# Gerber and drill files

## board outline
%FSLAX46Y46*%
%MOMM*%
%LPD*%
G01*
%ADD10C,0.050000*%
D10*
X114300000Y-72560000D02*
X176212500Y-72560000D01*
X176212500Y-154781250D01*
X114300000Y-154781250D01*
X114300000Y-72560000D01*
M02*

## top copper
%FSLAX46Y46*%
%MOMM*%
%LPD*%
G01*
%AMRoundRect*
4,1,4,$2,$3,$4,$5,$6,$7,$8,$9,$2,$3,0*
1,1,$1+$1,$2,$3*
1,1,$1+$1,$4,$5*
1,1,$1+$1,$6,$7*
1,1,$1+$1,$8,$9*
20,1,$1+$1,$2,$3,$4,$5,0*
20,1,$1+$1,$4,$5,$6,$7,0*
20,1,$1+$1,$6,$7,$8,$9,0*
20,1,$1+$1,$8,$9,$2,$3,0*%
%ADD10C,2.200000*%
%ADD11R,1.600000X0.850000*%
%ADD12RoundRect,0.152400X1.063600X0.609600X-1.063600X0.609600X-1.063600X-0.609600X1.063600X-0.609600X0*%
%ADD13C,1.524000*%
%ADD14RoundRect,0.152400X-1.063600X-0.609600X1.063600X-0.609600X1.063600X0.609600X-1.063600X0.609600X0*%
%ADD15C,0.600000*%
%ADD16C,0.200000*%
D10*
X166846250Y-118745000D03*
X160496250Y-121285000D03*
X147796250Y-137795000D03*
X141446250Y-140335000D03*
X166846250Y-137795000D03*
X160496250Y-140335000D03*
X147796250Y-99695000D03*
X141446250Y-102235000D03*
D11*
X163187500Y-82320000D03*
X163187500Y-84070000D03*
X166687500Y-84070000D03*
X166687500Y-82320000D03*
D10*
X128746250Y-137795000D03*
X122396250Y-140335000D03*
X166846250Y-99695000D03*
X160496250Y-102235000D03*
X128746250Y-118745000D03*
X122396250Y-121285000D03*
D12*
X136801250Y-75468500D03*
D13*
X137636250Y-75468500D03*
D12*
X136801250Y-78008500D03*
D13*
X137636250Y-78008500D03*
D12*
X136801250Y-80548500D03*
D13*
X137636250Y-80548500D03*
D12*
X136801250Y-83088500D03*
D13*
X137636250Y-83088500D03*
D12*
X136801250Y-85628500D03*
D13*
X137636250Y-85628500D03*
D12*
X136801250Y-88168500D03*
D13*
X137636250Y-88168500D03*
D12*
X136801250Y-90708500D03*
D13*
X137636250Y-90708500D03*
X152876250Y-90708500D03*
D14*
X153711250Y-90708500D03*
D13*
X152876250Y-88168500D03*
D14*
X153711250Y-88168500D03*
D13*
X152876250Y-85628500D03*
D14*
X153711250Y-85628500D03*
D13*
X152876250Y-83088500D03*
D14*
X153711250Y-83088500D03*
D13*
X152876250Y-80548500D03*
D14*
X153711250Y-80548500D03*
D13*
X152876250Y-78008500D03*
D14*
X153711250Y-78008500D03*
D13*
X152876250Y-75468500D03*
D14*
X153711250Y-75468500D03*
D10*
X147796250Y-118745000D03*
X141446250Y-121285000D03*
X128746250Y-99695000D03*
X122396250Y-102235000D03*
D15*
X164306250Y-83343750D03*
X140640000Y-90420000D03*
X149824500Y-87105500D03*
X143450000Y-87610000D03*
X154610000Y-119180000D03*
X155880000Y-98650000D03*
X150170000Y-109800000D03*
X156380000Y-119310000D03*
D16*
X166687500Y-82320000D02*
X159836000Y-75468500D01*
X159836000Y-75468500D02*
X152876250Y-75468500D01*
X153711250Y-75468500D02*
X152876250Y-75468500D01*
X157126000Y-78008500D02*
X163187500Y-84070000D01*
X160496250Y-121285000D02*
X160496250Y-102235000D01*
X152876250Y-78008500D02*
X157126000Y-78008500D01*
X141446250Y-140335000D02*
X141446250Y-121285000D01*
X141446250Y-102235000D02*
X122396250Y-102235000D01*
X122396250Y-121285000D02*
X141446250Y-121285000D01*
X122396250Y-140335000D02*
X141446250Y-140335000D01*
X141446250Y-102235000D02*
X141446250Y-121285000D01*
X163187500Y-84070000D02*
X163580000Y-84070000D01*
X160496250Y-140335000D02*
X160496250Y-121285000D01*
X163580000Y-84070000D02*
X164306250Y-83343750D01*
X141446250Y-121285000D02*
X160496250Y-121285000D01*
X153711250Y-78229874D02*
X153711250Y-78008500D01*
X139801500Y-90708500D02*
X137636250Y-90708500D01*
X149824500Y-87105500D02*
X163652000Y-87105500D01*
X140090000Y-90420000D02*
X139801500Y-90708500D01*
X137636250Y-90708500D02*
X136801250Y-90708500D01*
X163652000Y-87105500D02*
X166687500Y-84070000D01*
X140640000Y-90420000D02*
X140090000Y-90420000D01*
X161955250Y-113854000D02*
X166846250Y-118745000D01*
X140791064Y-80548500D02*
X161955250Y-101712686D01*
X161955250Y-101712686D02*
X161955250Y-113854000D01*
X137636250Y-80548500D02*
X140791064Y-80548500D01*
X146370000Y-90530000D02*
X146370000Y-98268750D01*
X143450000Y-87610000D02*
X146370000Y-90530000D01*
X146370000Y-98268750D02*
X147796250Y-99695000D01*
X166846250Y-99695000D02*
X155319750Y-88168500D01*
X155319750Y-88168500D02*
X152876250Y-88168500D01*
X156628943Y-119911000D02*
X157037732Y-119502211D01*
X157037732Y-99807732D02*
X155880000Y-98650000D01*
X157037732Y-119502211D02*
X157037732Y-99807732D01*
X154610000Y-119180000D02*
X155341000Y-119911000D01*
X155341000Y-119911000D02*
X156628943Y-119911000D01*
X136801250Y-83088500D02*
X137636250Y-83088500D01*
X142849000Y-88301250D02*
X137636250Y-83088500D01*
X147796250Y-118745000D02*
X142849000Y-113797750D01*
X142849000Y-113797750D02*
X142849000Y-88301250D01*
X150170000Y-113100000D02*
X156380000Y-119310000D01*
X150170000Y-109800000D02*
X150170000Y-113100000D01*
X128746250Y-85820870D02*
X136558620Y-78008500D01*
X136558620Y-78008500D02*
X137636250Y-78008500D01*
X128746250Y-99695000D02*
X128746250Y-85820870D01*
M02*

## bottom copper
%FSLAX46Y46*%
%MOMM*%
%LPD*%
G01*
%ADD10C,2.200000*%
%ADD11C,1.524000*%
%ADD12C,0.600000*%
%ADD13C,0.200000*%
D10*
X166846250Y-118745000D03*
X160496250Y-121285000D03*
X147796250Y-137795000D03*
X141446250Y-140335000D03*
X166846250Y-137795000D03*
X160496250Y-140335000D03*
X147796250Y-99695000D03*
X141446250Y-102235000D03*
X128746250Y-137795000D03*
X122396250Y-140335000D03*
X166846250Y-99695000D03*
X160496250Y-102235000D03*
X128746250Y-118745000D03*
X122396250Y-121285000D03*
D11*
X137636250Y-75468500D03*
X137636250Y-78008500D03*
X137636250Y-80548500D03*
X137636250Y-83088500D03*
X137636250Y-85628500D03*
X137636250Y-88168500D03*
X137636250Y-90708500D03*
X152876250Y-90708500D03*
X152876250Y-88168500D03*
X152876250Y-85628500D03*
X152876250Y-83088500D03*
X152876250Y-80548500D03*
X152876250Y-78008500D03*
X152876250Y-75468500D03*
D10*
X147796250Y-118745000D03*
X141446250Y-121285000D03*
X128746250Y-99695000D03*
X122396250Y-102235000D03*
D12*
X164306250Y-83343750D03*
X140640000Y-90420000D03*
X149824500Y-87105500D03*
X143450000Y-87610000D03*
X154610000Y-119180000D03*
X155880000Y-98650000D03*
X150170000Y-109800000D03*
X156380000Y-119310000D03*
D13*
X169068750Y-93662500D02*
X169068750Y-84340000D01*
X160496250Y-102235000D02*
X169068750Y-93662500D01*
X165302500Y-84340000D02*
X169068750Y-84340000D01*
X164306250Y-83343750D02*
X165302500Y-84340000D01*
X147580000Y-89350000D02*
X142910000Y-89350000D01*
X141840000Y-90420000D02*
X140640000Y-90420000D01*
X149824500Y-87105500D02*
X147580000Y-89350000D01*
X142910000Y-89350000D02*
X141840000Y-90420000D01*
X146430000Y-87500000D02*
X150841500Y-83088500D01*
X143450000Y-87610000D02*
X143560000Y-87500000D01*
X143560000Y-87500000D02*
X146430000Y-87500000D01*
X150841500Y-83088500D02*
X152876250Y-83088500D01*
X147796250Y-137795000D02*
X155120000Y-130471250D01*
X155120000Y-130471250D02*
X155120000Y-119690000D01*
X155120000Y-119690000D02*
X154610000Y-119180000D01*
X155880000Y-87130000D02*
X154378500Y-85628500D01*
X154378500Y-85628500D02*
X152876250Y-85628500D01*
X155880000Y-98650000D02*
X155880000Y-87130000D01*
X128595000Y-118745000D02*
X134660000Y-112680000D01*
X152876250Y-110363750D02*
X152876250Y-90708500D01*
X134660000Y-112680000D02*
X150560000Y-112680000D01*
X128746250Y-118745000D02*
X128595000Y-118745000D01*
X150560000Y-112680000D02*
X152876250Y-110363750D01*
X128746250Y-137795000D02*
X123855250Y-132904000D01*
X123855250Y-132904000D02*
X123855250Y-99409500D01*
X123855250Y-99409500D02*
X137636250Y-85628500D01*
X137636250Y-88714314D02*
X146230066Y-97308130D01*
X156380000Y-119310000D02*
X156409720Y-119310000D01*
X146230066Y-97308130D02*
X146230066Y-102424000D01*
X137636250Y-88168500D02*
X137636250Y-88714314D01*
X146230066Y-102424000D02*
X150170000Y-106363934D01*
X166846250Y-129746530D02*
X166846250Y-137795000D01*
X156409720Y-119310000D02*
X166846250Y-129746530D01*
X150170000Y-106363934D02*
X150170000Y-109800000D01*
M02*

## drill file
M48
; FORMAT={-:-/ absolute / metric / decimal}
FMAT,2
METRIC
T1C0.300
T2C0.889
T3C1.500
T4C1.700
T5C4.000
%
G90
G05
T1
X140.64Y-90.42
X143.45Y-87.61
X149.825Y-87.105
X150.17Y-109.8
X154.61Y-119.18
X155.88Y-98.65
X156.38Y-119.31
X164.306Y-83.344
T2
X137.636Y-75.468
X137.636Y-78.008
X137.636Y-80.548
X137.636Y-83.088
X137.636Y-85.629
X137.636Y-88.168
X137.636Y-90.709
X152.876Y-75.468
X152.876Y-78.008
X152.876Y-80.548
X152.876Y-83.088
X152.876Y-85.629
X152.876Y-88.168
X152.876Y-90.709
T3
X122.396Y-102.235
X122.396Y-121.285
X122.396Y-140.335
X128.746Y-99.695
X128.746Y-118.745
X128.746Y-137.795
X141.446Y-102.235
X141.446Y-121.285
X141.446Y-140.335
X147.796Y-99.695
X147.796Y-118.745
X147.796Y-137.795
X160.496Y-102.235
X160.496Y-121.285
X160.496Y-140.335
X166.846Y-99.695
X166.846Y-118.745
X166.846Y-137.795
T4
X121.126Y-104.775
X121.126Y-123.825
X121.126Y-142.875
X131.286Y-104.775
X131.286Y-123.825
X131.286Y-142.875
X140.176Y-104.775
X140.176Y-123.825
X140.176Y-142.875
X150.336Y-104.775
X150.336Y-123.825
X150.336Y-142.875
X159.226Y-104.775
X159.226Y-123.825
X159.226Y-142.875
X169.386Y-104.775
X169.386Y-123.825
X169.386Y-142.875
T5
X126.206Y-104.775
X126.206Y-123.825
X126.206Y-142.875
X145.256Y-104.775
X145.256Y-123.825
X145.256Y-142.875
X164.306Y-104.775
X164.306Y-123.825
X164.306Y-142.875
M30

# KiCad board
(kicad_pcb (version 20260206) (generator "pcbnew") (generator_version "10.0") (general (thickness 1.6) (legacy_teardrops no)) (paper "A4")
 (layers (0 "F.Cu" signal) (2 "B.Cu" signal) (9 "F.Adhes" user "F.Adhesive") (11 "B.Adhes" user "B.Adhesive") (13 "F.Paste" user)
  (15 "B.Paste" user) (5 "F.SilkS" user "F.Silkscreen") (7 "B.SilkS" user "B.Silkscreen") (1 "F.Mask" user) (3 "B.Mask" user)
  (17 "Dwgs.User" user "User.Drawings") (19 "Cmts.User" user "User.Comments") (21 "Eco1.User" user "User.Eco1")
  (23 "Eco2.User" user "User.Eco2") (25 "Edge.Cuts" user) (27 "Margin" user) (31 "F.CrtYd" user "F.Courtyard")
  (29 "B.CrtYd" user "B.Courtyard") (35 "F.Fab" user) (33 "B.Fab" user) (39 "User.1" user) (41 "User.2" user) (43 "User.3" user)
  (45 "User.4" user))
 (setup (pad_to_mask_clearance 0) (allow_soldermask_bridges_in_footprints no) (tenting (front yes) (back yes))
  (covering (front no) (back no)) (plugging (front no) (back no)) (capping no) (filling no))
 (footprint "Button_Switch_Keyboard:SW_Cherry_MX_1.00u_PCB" (layer "F.Cu") (at 166.84625 118.745)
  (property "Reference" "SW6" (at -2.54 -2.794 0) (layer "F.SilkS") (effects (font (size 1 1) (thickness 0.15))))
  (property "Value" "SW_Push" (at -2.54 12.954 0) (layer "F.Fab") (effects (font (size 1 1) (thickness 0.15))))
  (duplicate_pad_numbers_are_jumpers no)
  (pad "" np_thru_hole circle (at -7.62 5.08) (size 1.7 1.7) (drill 1.7) (layers "*.Cu" "*.Mask"))
  (pad "" np_thru_hole circle (at -2.54 5.08) (size 4 4) (drill 4) (layers "*.Cu" "*.Mask"))
  (pad "" np_thru_hole circle (at 2.54 5.08) (size 1.7 1.7) (drill 1.7) (layers "*.Cu" "*.Mask"))
  (pad "1" thru_hole circle (at 0 0) (size 2.2 2.2) (drill 1.5) (layers "*.Cu" "*.Mask") (remove_unused_layers no)
   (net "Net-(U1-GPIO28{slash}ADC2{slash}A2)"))
  (pad "2" thru_hole circle (at -6.35 2.54) (size 2.2 2.2) (drill 1.5) (layers "*.Cu" "*.Mask") (remove_unused_layers no) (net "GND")))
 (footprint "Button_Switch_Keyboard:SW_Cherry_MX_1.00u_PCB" (layer "F.Cu") (at 147.79625 137.795)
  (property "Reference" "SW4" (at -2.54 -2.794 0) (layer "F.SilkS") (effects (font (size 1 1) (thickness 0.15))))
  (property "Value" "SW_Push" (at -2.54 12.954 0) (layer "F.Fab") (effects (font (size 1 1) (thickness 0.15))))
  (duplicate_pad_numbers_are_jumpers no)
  (pad "" np_thru_hole circle (at -7.62 5.08) (size 1.7 1.7) (drill 1.7) (layers "*.Cu" "*.Mask"))
  (pad "" np_thru_hole circle (at -2.54 5.08) (size 4 4) (drill 4) (layers "*.Cu" "*.Mask"))
  (pad "" np_thru_hole circle (at 2.54 5.08) (size 1.7 1.7) (drill 1.7) (layers "*.Cu" "*.Mask"))
  (pad "1" thru_hole circle (at 0 0) (size 2.2 2.2) (drill 1.5) (layers "*.Cu" "*.Mask") (remove_unused_layers no)
   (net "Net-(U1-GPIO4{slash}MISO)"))
  (pad "2" thru_hole circle (at -6.35 2.54) (size 2.2 2.2) (drill 1.5) (layers "*.Cu" "*.Mask") (remove_unused_layers no) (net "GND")))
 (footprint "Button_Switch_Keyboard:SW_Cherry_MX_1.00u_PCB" (layer "F.Cu") (at 166.84625 137.795)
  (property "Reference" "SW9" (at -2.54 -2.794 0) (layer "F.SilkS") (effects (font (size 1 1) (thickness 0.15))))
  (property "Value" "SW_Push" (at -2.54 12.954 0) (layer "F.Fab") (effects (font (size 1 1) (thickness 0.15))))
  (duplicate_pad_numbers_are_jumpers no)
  (pad "" np_thru_hole circle (at -7.62 5.08) (size 1.7 1.7) (drill 1.7) (layers "*.Cu" "*.Mask"))
  (pad "" np_thru_hole circle (at -2.54 5.08) (size 4 4) (drill 4) (layers "*.Cu" "*.Mask"))
  (pad "" np_thru_hole circle (at 2.54 5.08) (size 1.7 1.7) (drill 1.7) (layers "*.Cu" "*.Mask"))
  (pad "1" thru_hole circle (at 0 0) (size 2.2 2.2) (drill 1.5) (layers "*.Cu" "*.Mask") (remove_unused_layers no)
   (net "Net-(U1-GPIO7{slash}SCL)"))
  (pad "2" thru_hole circle (at -6.35 2.54) (size 2.2 2.2) (drill 1.5) (layers "*.Cu" "*.Mask") (remove_unused_layers no) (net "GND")))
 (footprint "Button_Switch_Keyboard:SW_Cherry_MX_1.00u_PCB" (layer "F.Cu") (at 147.79625 99.695)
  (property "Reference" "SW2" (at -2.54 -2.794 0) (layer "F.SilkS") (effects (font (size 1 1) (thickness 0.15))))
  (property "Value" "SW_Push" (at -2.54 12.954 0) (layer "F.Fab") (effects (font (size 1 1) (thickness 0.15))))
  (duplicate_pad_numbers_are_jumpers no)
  (pad "" np_thru_hole circle (at -7.62 5.08) (size 1.7 1.7) (drill 1.7) (layers "*.Cu" "*.Mask"))
  (pad "" np_thru_hole circle (at -2.54 5.08) (size 4 4) (drill 4) (layers "*.Cu" "*.Mask"))
  (pad "" np_thru_hole circle (at 2.54 5.08) (size 1.7 1.7) (drill 1.7) (layers "*.Cu" "*.Mask"))
  (pad "1" thru_hole circle (at 0 0) (size 2.2 2.2) (drill 1.5) (layers "*.Cu" "*.Mask") (remove_unused_layers no)
   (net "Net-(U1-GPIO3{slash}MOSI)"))
  (pad "2" thru_hole circle (at -6.35 2.54) (size 2.2 2.2) (drill 1.5) (layers "*.Cu" "*.Mask") (remove_unused_layers no) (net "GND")))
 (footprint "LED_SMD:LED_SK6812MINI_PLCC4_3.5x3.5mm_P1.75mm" (layer "F.Cu") (at 164.9375 83.195)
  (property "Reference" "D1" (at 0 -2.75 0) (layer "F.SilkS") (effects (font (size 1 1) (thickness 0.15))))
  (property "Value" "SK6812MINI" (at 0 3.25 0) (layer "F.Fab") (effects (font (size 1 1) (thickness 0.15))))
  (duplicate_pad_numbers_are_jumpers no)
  (pad "1" smd rect (at -1.75 -0.875) (size 1.6 0.85) (layers "F.Cu" "F.Mask" "F.Paste") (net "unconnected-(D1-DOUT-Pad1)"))
  (pad "2" smd rect (at -1.75 0.875) (size 1.6 0.85) (layers "F.Cu" "F.Mask" "F.Paste") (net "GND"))
  (pad "3" smd rect (at 1.75 0.875) (size 1.6 0.85) (layers "F.Cu" "F.Mask" "F.Paste") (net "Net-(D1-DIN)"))
  (pad "4" smd rect (at 1.75 -0.875) (size 1.6 0.85) (layers "F.Cu" "F.Mask" "F.Paste") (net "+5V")))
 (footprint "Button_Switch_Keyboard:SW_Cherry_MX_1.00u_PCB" (layer "F.Cu") (at 128.74625 137.795)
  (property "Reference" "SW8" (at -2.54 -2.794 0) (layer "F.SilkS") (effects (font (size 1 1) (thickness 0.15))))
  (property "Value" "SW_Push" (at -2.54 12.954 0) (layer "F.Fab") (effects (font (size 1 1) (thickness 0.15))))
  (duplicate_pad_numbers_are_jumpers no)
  (pad "" np_thru_hole circle (at -7.62 5.08) (size 1.7 1.7) (drill 1.7) (layers "*.Cu" "*.Mask"))
  (pad "" np_thru_hole circle (at -2.54 5.08) (size 4 4) (drill 4) (layers "*.Cu" "*.Mask"))
  (pad "" np_thru_hole circle (at 2.54 5.08) (size 1.7 1.7) (drill 1.7) (layers "*.Cu" "*.Mask"))
  (pad "1" thru_hole circle (at 0 0) (size 2.2 2.2) (drill 1.5) (layers "*.Cu" "*.Mask") (remove_unused_layers no)
   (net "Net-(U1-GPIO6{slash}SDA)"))
  (pad "2" thru_hole circle (at -6.35 2.54) (size 2.2 2.2) (drill 1.5) (layers "*.Cu" "*.Mask") (remove_unused_layers no) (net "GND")))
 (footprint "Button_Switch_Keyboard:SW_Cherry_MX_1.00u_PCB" (layer "F.Cu") (at 166.84625 99.695)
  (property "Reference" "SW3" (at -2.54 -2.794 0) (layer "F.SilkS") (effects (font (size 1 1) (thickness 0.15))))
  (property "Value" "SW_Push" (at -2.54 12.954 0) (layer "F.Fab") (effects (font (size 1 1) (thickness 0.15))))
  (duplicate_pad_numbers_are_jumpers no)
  (pad "" np_thru_hole circle (at -7.62 5.08) (size 1.7 1.7) (drill 1.7) (layers "*.Cu" "*.Mask"))
  (pad "" np_thru_hole circle (at -2.54 5.08) (size 4 4) (drill 4) (layers "*.Cu" "*.Mask"))
  (pad "" np_thru_hole circle (at 2.54 5.08) (size 1.7 1.7) (drill 1.7) (layers "*.Cu" "*.Mask"))
  (pad "1" thru_hole circle (at 0 0) (size 2.2 2.2) (drill 1.5) (layers "*.Cu" "*.Mask") (remove_unused_layers no)
   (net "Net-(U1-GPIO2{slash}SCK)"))
  (pad "2" thru_hole circle (at -6.35 2.54) (size 2.2 2.2) (drill 1.5) (layers "*.Cu" "*.Mask") (remove_unused_layers no) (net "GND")))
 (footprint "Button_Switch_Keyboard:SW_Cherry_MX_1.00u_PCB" (layer "F.Cu") (at 128.74625 118.745)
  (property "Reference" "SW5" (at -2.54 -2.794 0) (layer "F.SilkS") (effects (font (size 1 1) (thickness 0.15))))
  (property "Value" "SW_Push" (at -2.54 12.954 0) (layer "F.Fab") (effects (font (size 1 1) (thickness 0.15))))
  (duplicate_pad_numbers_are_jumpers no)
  (pad "" np_thru_hole circle (at -7.62 5.08) (size 1.7 1.7) (drill 1.7) (layers "*.Cu" "*.Mask"))
  (pad "" np_thru_hole circle (at -2.54 5.08) (size 4 4) (drill 4) (layers "*.Cu" "*.Mask"))
  (pad "" np_thru_hole circle (at 2.54 5.08) (size 1.7 1.7) (drill 1.7) (layers "*.Cu" "*.Mask"))
  (pad "1" thru_hole circle (at 0 0) (size 2.2 2.2) (drill 1.5) (layers "*.Cu" "*.Mask") (remove_unused_layers no)
   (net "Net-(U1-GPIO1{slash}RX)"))
  (pad "2" thru_hole circle (at -6.35 2.54) (size 2.2 2.2) (drill 1.5) (layers "*.Cu" "*.Mask") (remove_unused_layers no) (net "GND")))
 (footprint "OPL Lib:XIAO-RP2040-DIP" (layer "F.Cu") (at 145.25625 83.0885)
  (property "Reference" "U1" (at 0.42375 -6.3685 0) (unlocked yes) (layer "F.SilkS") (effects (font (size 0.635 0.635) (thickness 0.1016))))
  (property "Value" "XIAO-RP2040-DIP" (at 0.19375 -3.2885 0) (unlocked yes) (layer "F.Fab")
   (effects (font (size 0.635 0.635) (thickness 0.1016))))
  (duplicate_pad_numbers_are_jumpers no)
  (pad "1" smd roundrect (at -8.455 -7.62 180) (size 2.432 1.524) (layers "F.Cu" "F.Mask") (roundrect_rratio 0.1)
   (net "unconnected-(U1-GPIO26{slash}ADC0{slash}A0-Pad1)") (thermal_bridge_angle 45))
  (pad "1" thru_hole circle (at -7.62 -7.62 180) (size 1.524 1.524) (drill 0.889) (layers "*.Cu" "*.Mask") (remove_unused_layers no)
   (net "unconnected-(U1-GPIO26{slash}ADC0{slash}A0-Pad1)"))
  (pad "2" smd roundrect (at -8.455 -5.08 180) (size 2.432 1.524) (layers "F.Cu" "F.Mask") (roundrect_rratio 0.1)
   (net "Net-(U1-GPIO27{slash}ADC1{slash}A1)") (thermal_bridge_angle 45))
  (pad "2" thru_hole circle (at -7.62 -5.08 180) (size 1.524 1.524) (drill 0.889) (layers "*.Cu" "*.Mask") (remove_unused_layers no)
   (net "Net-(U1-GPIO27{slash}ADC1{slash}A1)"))
  (pad "3" smd roundrect (at -8.455 -2.54 180) (size 2.432 1.524) (layers "F.Cu" "F.Mask") (roundrect_rratio 0.1)
   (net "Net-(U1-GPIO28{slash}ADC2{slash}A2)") (thermal_bridge_angle 45))
  (pad "3" thru_hole circle (at -7.62 -2.54 180) (size 1.524 1.524) (drill 0.889) (layers "*.Cu" "*.Mask") (remove_unused_layers no)
   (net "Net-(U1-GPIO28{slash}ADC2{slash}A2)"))
  (pad "4" smd roundrect (at -8.455 0 180) (size 2.432 1.524) (layers "F.Cu" "F.Mask") (roundrect_rratio 0.1)
   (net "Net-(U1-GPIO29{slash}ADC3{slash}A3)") (thermal_bridge_angle 45))
  (pad "4" thru_hole circle (at -7.62 0 180) (size 1.524 1.524) (drill 0.889) (layers "*.Cu" "*.Mask") (remove_unused_layers no)
   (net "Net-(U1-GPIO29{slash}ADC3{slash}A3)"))
  (pad "5" smd roundrect (at -8.455 2.54 180) (size 2.432 1.524) (layers "F.Cu" "F.Mask") (roundrect_rratio 0.1)
   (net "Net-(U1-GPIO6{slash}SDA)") (thermal_bridge_angle 45))
  (pad "5" thru_hole circle (at -7.62 2.54 180) (size 1.524 1.524) (drill 0.889) (layers "*.Cu" "*.Mask") (remove_unused_layers no)
   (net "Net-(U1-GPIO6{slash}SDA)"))
  (pad "6" smd roundrect (at -8.455 5.08 180) (size 2.432 1.524) (layers "F.Cu" "F.Mask") (roundrect_rratio 0.1)
   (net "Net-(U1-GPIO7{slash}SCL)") (thermal_bridge_angle 45))
  (pad "6" thru_hole circle (at -7.62 5.08 180) (size 1.524 1.524) (drill 0.889) (layers "*.Cu" "*.Mask") (remove_unused_layers no)
   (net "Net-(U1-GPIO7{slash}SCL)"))
  (pad "7" smd roundrect (at -8.455 7.62 180) (size 2.432 1.524) (layers "F.Cu" "F.Mask") (roundrect_rratio 0.1) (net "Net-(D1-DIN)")
   (thermal_bridge_angle 45))
  (pad "7" thru_hole circle (at -7.62 7.62 180) (size 1.524 1.524) (drill 0.889) (layers "*.Cu" "*.Mask") (remove_unused_layers no)
   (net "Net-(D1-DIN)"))
  (pad "8" thru_hole circle (at 7.62 7.62) (size 1.524 1.524) (drill 0.889) (layers "*.Cu" "*.Mask") (remove_unused_layers no)
   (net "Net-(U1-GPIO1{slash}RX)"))
  (pad "8" smd roundrect (at 8.455 7.62) (size 2.432 1.524) (layers "F.Cu" "F.Mask") (roundrect_rratio 0.1) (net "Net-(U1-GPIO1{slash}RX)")
   (thermal_bridge_angle 45))
  (pad "9" thru_hole circle (at 7.62 5.08) (size 1.524 1.524) (drill 0.889) (layers "*.Cu" "*.Mask") (remove_unused_layers no)
   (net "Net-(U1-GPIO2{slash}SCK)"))
  (pad "9" smd roundrect (at 8.455 5.08) (size 2.432 1.524) (layers "F.Cu" "F.Mask") (roundrect_rratio 0.1) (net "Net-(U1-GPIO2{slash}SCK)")
   (thermal_bridge_angle 45))
  (pad "10" thru_hole circle (at 7.62 2.54) (size 1.524 1.524) (drill 0.889) (layers "*.Cu" "*.Mask") (remove_unused_layers no)
   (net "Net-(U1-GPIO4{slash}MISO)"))
  (pad "10" smd roundrect (at 8.455 2.54) (size 2.432 1.524) (layers "F.Cu" "F.Mask") (roundrect_rratio 0.1)
   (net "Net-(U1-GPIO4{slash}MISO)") (thermal_bridge_angle 45))
  (pad "11" thru_hole circle (at 7.62 0) (size 1.524 1.524) (drill 0.889) (layers "*.Cu" "*.Mask") (remove_unused_layers no)
   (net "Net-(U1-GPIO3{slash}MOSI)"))
  (pad "11" smd roundrect (at 8.455 0) (size 2.432 1.524) (layers "F.Cu" "F.Mask") (roundrect_rratio 0.1) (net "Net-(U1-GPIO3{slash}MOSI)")
   (thermal_bridge_angle 45))
  (pad "12" thru_hole circle (at 7.62 -2.54) (size 1.524 1.524) (drill 0.889) (layers "*.Cu" "*.Mask") (remove_unused_layers no)
   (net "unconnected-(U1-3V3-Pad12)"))
  (pad "12" smd roundrect (at 8.455 -2.54) (size 2.432 1.524) (layers "F.Cu" "F.Mask") (roundrect_rratio 0.1)
   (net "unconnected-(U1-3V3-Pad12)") (thermal_bridge_angle 45))
  (pad "13" thru_hole circle (at 7.62 -5.08) (size 1.524 1.524) (drill 0.889) (layers "*.Cu" "*.Mask") (remove_unused_layers no) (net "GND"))
  (pad "13" smd roundrect (at 8.455 -5.08) (size 2.432 1.524) (layers "F.Cu" "F.Mask") (roundrect_rratio 0.1) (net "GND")
   (thermal_bridge_angle 45))
  (pad "14" thru_hole circle (at 7.62 -7.62) (size 1.524 1.524) (drill 0.889) (layers "*.Cu" "*.Mask") (remove_unused_layers no) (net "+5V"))
  (pad "14" smd roundrect (at 8.455 -7.62) (size 2.432 1.524) (layers "F.Cu" "F.Mask") (roundrect_rratio 0.1) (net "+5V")
   (thermal_bridge_angle 45)))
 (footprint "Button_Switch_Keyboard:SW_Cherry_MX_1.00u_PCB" (layer "F.Cu") (at 147.79625 118.745)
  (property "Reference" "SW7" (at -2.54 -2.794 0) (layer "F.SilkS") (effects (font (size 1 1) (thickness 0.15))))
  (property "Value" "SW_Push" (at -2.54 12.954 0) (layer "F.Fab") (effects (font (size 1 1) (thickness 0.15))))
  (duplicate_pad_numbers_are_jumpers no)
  (pad "" np_thru_hole circle (at -7.62 5.08) (size 1.7 1.7) (drill 1.7) (layers "*.Cu" "*.Mask"))
  (pad "" np_thru_hole circle (at -2.54 5.08) (size 4 4) (drill 4) (layers "*.Cu" "*.Mask"))
  (pad "" np_thru_hole circle (at 2.54 5.08) (size 1.7 1.7) (drill 1.7) (layers "*.Cu" "*.Mask"))
  (pad "1" thru_hole circle (at 0 0) (size 2.2 2.2) (drill 1.5) (layers "*.Cu" "*.Mask") (remove_unused_layers no)
   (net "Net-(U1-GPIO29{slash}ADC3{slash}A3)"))
  (pad "2" thru_hole circle (at -6.35 2.54) (size 2.2 2.2) (drill 1.5) (layers "*.Cu" "*.Mask") (remove_unused_layers no) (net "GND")))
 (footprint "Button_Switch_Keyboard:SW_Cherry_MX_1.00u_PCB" (layer "F.Cu") (at 128.74625 99.695)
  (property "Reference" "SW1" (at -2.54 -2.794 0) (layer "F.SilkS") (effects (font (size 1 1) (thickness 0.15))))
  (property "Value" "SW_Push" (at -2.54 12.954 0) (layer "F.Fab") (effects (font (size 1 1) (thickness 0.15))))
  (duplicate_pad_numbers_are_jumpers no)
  (pad "" np_thru_hole circle (at -7.62 5.08) (size 1.7 1.7) (drill 1.7) (layers "*.Cu" "*.Mask"))
  (pad "" np_thru_hole circle (at -2.54 5.08) (size 4 4) (drill 4) (layers "*.Cu" "*.Mask"))
  (pad "" np_thru_hole circle (at 2.54 5.08) (size 1.7 1.7) (drill 1.7) (layers "*.Cu" "*.Mask"))
  (pad "1" thru_hole circle (at 0 0) (size 2.2 2.2) (drill 1.5) (layers "*.Cu" "*.Mask") (remove_unused_layers no)
   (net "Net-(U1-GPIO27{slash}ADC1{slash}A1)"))
  (pad "2" thru_hole circle (at -6.35 2.54) (size 2.2 2.2) (drill 1.5) (layers "*.Cu" "*.Mask") (remove_unused_layers no) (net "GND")))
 (gr_rect (start 114.3 72.56) (end 176.2125 154.78125) (stroke (width 0.05) (type default)) (fill no) (layer "Edge.Cuts"))
 (segment (start 166.6875 82.32) (end 159.836 75.4685) (width 0.2) (layer "F.Cu") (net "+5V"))
 (segment (start 159.836 75.4685) (end 152.87625 75.4685) (width 0.2) (layer "F.Cu") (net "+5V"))
 (segment (start 153.71125 75.4685) (end 152.87625 75.4685) (width 0.2) (layer "F.Cu") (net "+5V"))
 (segment (start 157.126 78.0085) (end 163.1875 84.07) (width 0.2) (layer "F.Cu") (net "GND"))
 (segment (start 160.49625 121.285) (end 160.49625 102.235) (width 0.2) (layer "F.Cu") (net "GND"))
 (segment (start 152.87625 78.0085) (end 157.126 78.0085) (width 0.2) (layer "F.Cu") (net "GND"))
 (segment (start 141.44625 140.335) (end 141.44625 121.285) (width 0.2) (layer "F.Cu") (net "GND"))
 (segment (start 141.44625 102.235) (end 122.39625 102.235) (width 0.2) (layer "F.Cu") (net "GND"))
 (segment (start 122.39625 121.285) (end 141.44625 121.285) (width 0.2) (layer "F.Cu") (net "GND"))
 (segment (start 122.39625 140.335) (end 141.44625 140.335) (width 0.2) (layer "F.Cu") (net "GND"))
 (segment (start 141.44625 102.235) (end 141.44625 121.285) (width 0.2) (layer "F.Cu") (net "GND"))
 (segment (start 163.1875 84.07) (end 163.58 84.07) (width 0.2) (layer "F.Cu") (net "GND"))
 (segment (start 160.49625 140.335) (end 160.49625 121.285) (width 0.2) (layer "F.Cu") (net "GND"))
 (segment (start 163.58 84.07) (end 164.30625 83.34375) (width 0.2) (layer "F.Cu") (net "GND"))
 (segment (start 141.44625 121.285) (end 160.49625 121.285) (width 0.2) (layer "F.Cu") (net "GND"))
 (segment (start 153.71125 78.229874) (end 153.71125 78.0085) (width 0.2) (layer "F.Cu") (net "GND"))
 (via (at 164.30625 83.34375) (size 0.6) (drill 0.3) (layers "F.Cu" "B.Cu") (capping no) (covering (front no) (back no))
  (plugging (front no) (back no)) (filling no) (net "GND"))
 (segment (start 169.06875 93.6625) (end 169.06875 84.34) (width 0.2) (layer "B.Cu") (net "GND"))
 (segment (start 160.49625 102.235) (end 169.06875 93.6625) (width 0.2) (layer "B.Cu") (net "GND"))
 (segment (start 165.3025 84.34) (end 169.06875 84.34) (width 0.2) (layer "B.Cu") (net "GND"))
 (segment (start 164.30625 83.34375) (end 165.3025 84.34) (width 0.2) (layer "B.Cu") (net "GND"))
 (segment (start 139.8015 90.7085) (end 137.63625 90.7085) (width 0.2) (layer "F.Cu") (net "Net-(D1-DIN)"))
 (segment (start 149.8245 87.1055) (end 163.652 87.1055) (width 0.2) (layer "F.Cu") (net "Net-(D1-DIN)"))
 (segment (start 140.09 90.42) (end 139.8015 90.7085) (width 0.2) (layer "F.Cu") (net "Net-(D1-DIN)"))
 (segment (start 137.63625 90.7085) (end 136.80125 90.7085) (width 0.2) (layer "F.Cu") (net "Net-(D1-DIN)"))
 (segment (start 163.652 87.1055) (end 166.6875 84.07) (width 0.2) (layer "F.Cu") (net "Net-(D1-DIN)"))
 (segment (start 140.64 90.42) (end 140.09 90.42) (width 0.2) (layer "F.Cu") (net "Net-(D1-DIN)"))
 (via (at 140.64 90.42) (size 0.6) (drill 0.3) (layers "F.Cu" "B.Cu") (capping no) (covering (front no) (back no))
  (plugging (front no) (back no)) (filling no) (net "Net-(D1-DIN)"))
 (via (at 149.8245 87.1055) (size 0.6) (drill 0.3) (layers "F.Cu" "B.Cu") (capping no) (covering (front no) (back no))
  (plugging (front no) (back no)) (filling no) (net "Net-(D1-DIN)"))
 (segment (start 147.58 89.35) (end 142.91 89.35) (width 0.2) (layer "B.Cu") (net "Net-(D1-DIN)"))
 (segment (start 141.84 90.42) (end 140.64 90.42) (width 0.2) (layer "B.Cu") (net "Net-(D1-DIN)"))
 (segment (start 149.8245 87.1055) (end 147.58 89.35) (width 0.2) (layer "B.Cu") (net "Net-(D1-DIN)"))
 (segment (start 142.91 89.35) (end 141.84 90.42) (width 0.2) (layer "B.Cu") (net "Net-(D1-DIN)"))
 (segment (start 161.95525 113.854) (end 166.84625 118.745) (width 0.2) (layer "F.Cu") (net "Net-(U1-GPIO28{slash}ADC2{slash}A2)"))
 (segment (start 140.791064 80.5485) (end 161.95525 101.712686) (width 0.2) (layer "F.Cu") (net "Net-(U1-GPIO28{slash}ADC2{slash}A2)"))
 (segment (start 161.95525 101.712686) (end 161.95525 113.854) (width 0.2) (layer "F.Cu") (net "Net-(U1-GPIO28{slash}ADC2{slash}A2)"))
 (segment (start 137.63625 80.5485) (end 140.791064 80.5485) (width 0.2) (layer "F.Cu") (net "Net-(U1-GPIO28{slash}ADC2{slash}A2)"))
 (segment (start 146.37 90.53) (end 146.37 98.26875) (width 0.2) (layer "F.Cu") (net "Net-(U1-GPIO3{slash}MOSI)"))
 (segment (start 143.45 87.61) (end 146.37 90.53) (width 0.2) (layer "F.Cu") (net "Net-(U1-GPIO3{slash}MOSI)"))
 (segment (start 146.37 98.26875) (end 147.79625 99.695) (width 0.2) (layer "F.Cu") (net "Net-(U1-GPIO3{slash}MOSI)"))
 (via (at 143.45 87.61) (size 0.6) (drill 0.3) (layers "F.Cu" "B.Cu") (capping no) (covering (front no) (back no))
  (plugging (front no) (back no)) (filling no) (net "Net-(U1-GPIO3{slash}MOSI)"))
 (segment (start 146.43 87.5) (end 150.8415 83.0885) (width 0.2) (layer "B.Cu") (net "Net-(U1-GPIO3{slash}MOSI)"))
 (segment (start 143.45 87.61) (end 143.56 87.5) (width 0.2) (layer "B.Cu") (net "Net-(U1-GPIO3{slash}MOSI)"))
 (segment (start 143.56 87.5) (end 146.43 87.5) (width 0.2) (layer "B.Cu") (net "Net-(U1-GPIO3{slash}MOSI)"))
 (segment (start 150.8415 83.0885) (end 152.87625 83.0885) (width 0.2) (layer "B.Cu") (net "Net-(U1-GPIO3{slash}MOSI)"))
 (segment (start 166.84625 99.695) (end 155.31975 88.1685) (width 0.2) (layer "F.Cu") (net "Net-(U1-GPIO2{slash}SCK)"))
 (segment (start 155.31975 88.1685) (end 152.87625 88.1685) (width 0.2) (layer "F.Cu") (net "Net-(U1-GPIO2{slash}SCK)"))
 (segment (start 156.628943 119.911) (end 157.037732 119.502211) (width 0.2) (layer "F.Cu") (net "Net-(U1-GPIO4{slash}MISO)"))
 (segment (start 157.037732 99.807732) (end 155.88 98.65) (width 0.2) (layer "F.Cu") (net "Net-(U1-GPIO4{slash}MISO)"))
 (segment (start 157.037732 119.502211) (end 157.037732 99.807732) (width 0.2) (layer "F.Cu") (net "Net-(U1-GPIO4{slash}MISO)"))
 (segment (start 154.61 119.18) (end 155.341 119.911) (width 0.2) (layer "F.Cu") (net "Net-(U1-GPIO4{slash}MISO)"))
 (segment (start 155.341 119.911) (end 156.628943 119.911) (width 0.2) (layer "F.Cu") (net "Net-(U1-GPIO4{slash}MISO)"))
 (via (at 154.61 119.18) (size 0.6) (drill 0.3) (layers "F.Cu" "B.Cu") (capping no) (covering (front no) (back no))
  (plugging (front no) (back no)) (filling no) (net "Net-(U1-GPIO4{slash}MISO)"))
 (via (at 155.88 98.65) (size 0.6) (drill 0.3) (layers "F.Cu" "B.Cu") (capping no) (covering (front no) (back no))
  (plugging (front no) (back no)) (filling no) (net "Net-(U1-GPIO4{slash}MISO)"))
 (segment (start 147.79625 137.795) (end 155.12 130.47125) (width 0.2) (layer "B.Cu") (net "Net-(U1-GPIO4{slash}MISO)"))
 (segment (start 155.12 130.47125) (end 155.12 119.69) (width 0.2) (layer "B.Cu") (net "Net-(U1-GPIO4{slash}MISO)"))
 (segment (start 155.12 119.69) (end 154.61 119.18) (width 0.2) (layer "B.Cu") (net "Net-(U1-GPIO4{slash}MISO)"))
 (segment (start 155.88 87.13) (end 154.3785 85.6285) (width 0.2) (layer "B.Cu") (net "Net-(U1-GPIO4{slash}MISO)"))
 (segment (start 154.3785 85.6285) (end 152.87625 85.6285) (width 0.2) (layer "B.Cu") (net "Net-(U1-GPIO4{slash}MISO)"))
 (segment (start 155.88 98.65) (end 155.88 87.13) (width 0.2) (layer "B.Cu") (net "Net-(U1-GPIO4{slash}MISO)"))
 (segment (start 128.595 118.745) (end 134.66 112.68) (width 0.2) (layer "B.Cu") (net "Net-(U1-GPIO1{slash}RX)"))
 (segment (start 152.87625 110.36375) (end 152.87625 90.7085) (width 0.2) (layer "B.Cu") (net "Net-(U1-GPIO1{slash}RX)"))
 (segment (start 134.66 112.68) (end 150.56 112.68) (width 0.2) (layer "B.Cu") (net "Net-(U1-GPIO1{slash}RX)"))
 (segment (start 128.74625 118.745) (end 128.595 118.745) (width 0.2) (layer "B.Cu") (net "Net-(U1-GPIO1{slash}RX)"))
 (segment (start 150.56 112.68) (end 152.87625 110.36375) (width 0.2) (layer "B.Cu") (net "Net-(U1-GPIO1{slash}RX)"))
 (segment (start 136.80125 83.0885) (end 137.63625 83.0885) (width 0.2) (layer "F.Cu") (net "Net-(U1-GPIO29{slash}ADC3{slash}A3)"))
 (segment (start 142.849 88.30125) (end 137.63625 83.0885) (width 0.2) (layer "F.Cu") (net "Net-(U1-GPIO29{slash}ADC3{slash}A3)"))
 (segment (start 147.79625 118.745) (end 142.849 113.79775) (width 0.2) (layer "F.Cu") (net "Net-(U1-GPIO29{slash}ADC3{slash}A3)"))
 (segment (start 142.849 113.79775) (end 142.849 88.30125) (width 0.2) (layer "F.Cu") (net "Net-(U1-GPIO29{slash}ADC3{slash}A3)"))
 (segment (start 128.74625 137.795) (end 123.85525 132.904) (width 0.2) (layer "B.Cu") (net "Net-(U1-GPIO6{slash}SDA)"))
 (segment (start 123.85525 132.904) (end 123.85525 99.4095) (width 0.2) (layer "B.Cu") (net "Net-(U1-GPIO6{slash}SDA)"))
 (segment (start 123.85525 99.4095) (end 137.63625 85.6285) (width 0.2) (layer "B.Cu") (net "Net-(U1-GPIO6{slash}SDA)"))
 (segment (start 150.17 113.1) (end 156.38 119.31) (width 0.2) (layer "F.Cu") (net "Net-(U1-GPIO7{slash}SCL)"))
 (segment (start 150.17 109.8) (end 150.17 113.1) (width 0.2) (layer "F.Cu") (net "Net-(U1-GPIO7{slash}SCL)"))
 (via (at 150.17 109.8) (size 0.6) (drill 0.3) (layers "F.Cu" "B.Cu") (capping no) (covering (front no) (back no))
  (plugging (front no) (back no)) (filling no) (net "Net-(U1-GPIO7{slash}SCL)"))
 (via (at 156.38 119.31) (size 0.6) (drill 0.3) (layers "F.Cu" "B.Cu") (capping no) (covering (front no) (back no))
  (plugging (front no) (back no)) (filling no) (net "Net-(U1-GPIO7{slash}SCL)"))
 (segment (start 137.63625 88.714314) (end 146.230066 97.30813) (width 0.2) (layer "B.Cu") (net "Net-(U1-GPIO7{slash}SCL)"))
 (segment (start 156.38 119.31) (end 156.40972 119.31) (width 0.2) (layer "B.Cu") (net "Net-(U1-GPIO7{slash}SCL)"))
 (segment (start 146.230066 97.30813) (end 146.230066 102.424) (width 0.2) (layer "B.Cu") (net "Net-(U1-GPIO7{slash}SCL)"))
 (segment (start 137.63625 88.1685) (end 137.63625 88.714314) (width 0.2) (layer "B.Cu") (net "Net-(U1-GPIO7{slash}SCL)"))
 (segment (start 146.230066 102.424) (end 150.17 106.363934) (width 0.2) (layer "B.Cu") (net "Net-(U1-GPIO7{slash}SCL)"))
 (segment (start 166.84625 129.74653) (end 166.84625 137.795) (width 0.2) (layer "B.Cu") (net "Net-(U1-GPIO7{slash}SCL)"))
 (segment (start 156.40972 119.31) (end 166.84625 129.74653) (width 0.2) (layer "B.Cu") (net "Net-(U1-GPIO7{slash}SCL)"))
 (segment (start 150.17 106.363934) (end 150.17 109.8) (width 0.2) (layer "B.Cu") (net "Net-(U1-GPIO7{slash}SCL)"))
 (segment (start 128.74625 85.82087) (end 136.55862 78.0085) (width 0.2) (layer "F.Cu") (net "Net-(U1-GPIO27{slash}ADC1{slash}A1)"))
 (segment (start 136.55862 78.0085) (end 137.63625 78.0085) (width 0.2) (layer "F.Cu") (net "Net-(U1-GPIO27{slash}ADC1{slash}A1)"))
 (segment (start 128.74625 99.695) (end 128.74625 85.82087) (width 0.2) (layer "F.Cu") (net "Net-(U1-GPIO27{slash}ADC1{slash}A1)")))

